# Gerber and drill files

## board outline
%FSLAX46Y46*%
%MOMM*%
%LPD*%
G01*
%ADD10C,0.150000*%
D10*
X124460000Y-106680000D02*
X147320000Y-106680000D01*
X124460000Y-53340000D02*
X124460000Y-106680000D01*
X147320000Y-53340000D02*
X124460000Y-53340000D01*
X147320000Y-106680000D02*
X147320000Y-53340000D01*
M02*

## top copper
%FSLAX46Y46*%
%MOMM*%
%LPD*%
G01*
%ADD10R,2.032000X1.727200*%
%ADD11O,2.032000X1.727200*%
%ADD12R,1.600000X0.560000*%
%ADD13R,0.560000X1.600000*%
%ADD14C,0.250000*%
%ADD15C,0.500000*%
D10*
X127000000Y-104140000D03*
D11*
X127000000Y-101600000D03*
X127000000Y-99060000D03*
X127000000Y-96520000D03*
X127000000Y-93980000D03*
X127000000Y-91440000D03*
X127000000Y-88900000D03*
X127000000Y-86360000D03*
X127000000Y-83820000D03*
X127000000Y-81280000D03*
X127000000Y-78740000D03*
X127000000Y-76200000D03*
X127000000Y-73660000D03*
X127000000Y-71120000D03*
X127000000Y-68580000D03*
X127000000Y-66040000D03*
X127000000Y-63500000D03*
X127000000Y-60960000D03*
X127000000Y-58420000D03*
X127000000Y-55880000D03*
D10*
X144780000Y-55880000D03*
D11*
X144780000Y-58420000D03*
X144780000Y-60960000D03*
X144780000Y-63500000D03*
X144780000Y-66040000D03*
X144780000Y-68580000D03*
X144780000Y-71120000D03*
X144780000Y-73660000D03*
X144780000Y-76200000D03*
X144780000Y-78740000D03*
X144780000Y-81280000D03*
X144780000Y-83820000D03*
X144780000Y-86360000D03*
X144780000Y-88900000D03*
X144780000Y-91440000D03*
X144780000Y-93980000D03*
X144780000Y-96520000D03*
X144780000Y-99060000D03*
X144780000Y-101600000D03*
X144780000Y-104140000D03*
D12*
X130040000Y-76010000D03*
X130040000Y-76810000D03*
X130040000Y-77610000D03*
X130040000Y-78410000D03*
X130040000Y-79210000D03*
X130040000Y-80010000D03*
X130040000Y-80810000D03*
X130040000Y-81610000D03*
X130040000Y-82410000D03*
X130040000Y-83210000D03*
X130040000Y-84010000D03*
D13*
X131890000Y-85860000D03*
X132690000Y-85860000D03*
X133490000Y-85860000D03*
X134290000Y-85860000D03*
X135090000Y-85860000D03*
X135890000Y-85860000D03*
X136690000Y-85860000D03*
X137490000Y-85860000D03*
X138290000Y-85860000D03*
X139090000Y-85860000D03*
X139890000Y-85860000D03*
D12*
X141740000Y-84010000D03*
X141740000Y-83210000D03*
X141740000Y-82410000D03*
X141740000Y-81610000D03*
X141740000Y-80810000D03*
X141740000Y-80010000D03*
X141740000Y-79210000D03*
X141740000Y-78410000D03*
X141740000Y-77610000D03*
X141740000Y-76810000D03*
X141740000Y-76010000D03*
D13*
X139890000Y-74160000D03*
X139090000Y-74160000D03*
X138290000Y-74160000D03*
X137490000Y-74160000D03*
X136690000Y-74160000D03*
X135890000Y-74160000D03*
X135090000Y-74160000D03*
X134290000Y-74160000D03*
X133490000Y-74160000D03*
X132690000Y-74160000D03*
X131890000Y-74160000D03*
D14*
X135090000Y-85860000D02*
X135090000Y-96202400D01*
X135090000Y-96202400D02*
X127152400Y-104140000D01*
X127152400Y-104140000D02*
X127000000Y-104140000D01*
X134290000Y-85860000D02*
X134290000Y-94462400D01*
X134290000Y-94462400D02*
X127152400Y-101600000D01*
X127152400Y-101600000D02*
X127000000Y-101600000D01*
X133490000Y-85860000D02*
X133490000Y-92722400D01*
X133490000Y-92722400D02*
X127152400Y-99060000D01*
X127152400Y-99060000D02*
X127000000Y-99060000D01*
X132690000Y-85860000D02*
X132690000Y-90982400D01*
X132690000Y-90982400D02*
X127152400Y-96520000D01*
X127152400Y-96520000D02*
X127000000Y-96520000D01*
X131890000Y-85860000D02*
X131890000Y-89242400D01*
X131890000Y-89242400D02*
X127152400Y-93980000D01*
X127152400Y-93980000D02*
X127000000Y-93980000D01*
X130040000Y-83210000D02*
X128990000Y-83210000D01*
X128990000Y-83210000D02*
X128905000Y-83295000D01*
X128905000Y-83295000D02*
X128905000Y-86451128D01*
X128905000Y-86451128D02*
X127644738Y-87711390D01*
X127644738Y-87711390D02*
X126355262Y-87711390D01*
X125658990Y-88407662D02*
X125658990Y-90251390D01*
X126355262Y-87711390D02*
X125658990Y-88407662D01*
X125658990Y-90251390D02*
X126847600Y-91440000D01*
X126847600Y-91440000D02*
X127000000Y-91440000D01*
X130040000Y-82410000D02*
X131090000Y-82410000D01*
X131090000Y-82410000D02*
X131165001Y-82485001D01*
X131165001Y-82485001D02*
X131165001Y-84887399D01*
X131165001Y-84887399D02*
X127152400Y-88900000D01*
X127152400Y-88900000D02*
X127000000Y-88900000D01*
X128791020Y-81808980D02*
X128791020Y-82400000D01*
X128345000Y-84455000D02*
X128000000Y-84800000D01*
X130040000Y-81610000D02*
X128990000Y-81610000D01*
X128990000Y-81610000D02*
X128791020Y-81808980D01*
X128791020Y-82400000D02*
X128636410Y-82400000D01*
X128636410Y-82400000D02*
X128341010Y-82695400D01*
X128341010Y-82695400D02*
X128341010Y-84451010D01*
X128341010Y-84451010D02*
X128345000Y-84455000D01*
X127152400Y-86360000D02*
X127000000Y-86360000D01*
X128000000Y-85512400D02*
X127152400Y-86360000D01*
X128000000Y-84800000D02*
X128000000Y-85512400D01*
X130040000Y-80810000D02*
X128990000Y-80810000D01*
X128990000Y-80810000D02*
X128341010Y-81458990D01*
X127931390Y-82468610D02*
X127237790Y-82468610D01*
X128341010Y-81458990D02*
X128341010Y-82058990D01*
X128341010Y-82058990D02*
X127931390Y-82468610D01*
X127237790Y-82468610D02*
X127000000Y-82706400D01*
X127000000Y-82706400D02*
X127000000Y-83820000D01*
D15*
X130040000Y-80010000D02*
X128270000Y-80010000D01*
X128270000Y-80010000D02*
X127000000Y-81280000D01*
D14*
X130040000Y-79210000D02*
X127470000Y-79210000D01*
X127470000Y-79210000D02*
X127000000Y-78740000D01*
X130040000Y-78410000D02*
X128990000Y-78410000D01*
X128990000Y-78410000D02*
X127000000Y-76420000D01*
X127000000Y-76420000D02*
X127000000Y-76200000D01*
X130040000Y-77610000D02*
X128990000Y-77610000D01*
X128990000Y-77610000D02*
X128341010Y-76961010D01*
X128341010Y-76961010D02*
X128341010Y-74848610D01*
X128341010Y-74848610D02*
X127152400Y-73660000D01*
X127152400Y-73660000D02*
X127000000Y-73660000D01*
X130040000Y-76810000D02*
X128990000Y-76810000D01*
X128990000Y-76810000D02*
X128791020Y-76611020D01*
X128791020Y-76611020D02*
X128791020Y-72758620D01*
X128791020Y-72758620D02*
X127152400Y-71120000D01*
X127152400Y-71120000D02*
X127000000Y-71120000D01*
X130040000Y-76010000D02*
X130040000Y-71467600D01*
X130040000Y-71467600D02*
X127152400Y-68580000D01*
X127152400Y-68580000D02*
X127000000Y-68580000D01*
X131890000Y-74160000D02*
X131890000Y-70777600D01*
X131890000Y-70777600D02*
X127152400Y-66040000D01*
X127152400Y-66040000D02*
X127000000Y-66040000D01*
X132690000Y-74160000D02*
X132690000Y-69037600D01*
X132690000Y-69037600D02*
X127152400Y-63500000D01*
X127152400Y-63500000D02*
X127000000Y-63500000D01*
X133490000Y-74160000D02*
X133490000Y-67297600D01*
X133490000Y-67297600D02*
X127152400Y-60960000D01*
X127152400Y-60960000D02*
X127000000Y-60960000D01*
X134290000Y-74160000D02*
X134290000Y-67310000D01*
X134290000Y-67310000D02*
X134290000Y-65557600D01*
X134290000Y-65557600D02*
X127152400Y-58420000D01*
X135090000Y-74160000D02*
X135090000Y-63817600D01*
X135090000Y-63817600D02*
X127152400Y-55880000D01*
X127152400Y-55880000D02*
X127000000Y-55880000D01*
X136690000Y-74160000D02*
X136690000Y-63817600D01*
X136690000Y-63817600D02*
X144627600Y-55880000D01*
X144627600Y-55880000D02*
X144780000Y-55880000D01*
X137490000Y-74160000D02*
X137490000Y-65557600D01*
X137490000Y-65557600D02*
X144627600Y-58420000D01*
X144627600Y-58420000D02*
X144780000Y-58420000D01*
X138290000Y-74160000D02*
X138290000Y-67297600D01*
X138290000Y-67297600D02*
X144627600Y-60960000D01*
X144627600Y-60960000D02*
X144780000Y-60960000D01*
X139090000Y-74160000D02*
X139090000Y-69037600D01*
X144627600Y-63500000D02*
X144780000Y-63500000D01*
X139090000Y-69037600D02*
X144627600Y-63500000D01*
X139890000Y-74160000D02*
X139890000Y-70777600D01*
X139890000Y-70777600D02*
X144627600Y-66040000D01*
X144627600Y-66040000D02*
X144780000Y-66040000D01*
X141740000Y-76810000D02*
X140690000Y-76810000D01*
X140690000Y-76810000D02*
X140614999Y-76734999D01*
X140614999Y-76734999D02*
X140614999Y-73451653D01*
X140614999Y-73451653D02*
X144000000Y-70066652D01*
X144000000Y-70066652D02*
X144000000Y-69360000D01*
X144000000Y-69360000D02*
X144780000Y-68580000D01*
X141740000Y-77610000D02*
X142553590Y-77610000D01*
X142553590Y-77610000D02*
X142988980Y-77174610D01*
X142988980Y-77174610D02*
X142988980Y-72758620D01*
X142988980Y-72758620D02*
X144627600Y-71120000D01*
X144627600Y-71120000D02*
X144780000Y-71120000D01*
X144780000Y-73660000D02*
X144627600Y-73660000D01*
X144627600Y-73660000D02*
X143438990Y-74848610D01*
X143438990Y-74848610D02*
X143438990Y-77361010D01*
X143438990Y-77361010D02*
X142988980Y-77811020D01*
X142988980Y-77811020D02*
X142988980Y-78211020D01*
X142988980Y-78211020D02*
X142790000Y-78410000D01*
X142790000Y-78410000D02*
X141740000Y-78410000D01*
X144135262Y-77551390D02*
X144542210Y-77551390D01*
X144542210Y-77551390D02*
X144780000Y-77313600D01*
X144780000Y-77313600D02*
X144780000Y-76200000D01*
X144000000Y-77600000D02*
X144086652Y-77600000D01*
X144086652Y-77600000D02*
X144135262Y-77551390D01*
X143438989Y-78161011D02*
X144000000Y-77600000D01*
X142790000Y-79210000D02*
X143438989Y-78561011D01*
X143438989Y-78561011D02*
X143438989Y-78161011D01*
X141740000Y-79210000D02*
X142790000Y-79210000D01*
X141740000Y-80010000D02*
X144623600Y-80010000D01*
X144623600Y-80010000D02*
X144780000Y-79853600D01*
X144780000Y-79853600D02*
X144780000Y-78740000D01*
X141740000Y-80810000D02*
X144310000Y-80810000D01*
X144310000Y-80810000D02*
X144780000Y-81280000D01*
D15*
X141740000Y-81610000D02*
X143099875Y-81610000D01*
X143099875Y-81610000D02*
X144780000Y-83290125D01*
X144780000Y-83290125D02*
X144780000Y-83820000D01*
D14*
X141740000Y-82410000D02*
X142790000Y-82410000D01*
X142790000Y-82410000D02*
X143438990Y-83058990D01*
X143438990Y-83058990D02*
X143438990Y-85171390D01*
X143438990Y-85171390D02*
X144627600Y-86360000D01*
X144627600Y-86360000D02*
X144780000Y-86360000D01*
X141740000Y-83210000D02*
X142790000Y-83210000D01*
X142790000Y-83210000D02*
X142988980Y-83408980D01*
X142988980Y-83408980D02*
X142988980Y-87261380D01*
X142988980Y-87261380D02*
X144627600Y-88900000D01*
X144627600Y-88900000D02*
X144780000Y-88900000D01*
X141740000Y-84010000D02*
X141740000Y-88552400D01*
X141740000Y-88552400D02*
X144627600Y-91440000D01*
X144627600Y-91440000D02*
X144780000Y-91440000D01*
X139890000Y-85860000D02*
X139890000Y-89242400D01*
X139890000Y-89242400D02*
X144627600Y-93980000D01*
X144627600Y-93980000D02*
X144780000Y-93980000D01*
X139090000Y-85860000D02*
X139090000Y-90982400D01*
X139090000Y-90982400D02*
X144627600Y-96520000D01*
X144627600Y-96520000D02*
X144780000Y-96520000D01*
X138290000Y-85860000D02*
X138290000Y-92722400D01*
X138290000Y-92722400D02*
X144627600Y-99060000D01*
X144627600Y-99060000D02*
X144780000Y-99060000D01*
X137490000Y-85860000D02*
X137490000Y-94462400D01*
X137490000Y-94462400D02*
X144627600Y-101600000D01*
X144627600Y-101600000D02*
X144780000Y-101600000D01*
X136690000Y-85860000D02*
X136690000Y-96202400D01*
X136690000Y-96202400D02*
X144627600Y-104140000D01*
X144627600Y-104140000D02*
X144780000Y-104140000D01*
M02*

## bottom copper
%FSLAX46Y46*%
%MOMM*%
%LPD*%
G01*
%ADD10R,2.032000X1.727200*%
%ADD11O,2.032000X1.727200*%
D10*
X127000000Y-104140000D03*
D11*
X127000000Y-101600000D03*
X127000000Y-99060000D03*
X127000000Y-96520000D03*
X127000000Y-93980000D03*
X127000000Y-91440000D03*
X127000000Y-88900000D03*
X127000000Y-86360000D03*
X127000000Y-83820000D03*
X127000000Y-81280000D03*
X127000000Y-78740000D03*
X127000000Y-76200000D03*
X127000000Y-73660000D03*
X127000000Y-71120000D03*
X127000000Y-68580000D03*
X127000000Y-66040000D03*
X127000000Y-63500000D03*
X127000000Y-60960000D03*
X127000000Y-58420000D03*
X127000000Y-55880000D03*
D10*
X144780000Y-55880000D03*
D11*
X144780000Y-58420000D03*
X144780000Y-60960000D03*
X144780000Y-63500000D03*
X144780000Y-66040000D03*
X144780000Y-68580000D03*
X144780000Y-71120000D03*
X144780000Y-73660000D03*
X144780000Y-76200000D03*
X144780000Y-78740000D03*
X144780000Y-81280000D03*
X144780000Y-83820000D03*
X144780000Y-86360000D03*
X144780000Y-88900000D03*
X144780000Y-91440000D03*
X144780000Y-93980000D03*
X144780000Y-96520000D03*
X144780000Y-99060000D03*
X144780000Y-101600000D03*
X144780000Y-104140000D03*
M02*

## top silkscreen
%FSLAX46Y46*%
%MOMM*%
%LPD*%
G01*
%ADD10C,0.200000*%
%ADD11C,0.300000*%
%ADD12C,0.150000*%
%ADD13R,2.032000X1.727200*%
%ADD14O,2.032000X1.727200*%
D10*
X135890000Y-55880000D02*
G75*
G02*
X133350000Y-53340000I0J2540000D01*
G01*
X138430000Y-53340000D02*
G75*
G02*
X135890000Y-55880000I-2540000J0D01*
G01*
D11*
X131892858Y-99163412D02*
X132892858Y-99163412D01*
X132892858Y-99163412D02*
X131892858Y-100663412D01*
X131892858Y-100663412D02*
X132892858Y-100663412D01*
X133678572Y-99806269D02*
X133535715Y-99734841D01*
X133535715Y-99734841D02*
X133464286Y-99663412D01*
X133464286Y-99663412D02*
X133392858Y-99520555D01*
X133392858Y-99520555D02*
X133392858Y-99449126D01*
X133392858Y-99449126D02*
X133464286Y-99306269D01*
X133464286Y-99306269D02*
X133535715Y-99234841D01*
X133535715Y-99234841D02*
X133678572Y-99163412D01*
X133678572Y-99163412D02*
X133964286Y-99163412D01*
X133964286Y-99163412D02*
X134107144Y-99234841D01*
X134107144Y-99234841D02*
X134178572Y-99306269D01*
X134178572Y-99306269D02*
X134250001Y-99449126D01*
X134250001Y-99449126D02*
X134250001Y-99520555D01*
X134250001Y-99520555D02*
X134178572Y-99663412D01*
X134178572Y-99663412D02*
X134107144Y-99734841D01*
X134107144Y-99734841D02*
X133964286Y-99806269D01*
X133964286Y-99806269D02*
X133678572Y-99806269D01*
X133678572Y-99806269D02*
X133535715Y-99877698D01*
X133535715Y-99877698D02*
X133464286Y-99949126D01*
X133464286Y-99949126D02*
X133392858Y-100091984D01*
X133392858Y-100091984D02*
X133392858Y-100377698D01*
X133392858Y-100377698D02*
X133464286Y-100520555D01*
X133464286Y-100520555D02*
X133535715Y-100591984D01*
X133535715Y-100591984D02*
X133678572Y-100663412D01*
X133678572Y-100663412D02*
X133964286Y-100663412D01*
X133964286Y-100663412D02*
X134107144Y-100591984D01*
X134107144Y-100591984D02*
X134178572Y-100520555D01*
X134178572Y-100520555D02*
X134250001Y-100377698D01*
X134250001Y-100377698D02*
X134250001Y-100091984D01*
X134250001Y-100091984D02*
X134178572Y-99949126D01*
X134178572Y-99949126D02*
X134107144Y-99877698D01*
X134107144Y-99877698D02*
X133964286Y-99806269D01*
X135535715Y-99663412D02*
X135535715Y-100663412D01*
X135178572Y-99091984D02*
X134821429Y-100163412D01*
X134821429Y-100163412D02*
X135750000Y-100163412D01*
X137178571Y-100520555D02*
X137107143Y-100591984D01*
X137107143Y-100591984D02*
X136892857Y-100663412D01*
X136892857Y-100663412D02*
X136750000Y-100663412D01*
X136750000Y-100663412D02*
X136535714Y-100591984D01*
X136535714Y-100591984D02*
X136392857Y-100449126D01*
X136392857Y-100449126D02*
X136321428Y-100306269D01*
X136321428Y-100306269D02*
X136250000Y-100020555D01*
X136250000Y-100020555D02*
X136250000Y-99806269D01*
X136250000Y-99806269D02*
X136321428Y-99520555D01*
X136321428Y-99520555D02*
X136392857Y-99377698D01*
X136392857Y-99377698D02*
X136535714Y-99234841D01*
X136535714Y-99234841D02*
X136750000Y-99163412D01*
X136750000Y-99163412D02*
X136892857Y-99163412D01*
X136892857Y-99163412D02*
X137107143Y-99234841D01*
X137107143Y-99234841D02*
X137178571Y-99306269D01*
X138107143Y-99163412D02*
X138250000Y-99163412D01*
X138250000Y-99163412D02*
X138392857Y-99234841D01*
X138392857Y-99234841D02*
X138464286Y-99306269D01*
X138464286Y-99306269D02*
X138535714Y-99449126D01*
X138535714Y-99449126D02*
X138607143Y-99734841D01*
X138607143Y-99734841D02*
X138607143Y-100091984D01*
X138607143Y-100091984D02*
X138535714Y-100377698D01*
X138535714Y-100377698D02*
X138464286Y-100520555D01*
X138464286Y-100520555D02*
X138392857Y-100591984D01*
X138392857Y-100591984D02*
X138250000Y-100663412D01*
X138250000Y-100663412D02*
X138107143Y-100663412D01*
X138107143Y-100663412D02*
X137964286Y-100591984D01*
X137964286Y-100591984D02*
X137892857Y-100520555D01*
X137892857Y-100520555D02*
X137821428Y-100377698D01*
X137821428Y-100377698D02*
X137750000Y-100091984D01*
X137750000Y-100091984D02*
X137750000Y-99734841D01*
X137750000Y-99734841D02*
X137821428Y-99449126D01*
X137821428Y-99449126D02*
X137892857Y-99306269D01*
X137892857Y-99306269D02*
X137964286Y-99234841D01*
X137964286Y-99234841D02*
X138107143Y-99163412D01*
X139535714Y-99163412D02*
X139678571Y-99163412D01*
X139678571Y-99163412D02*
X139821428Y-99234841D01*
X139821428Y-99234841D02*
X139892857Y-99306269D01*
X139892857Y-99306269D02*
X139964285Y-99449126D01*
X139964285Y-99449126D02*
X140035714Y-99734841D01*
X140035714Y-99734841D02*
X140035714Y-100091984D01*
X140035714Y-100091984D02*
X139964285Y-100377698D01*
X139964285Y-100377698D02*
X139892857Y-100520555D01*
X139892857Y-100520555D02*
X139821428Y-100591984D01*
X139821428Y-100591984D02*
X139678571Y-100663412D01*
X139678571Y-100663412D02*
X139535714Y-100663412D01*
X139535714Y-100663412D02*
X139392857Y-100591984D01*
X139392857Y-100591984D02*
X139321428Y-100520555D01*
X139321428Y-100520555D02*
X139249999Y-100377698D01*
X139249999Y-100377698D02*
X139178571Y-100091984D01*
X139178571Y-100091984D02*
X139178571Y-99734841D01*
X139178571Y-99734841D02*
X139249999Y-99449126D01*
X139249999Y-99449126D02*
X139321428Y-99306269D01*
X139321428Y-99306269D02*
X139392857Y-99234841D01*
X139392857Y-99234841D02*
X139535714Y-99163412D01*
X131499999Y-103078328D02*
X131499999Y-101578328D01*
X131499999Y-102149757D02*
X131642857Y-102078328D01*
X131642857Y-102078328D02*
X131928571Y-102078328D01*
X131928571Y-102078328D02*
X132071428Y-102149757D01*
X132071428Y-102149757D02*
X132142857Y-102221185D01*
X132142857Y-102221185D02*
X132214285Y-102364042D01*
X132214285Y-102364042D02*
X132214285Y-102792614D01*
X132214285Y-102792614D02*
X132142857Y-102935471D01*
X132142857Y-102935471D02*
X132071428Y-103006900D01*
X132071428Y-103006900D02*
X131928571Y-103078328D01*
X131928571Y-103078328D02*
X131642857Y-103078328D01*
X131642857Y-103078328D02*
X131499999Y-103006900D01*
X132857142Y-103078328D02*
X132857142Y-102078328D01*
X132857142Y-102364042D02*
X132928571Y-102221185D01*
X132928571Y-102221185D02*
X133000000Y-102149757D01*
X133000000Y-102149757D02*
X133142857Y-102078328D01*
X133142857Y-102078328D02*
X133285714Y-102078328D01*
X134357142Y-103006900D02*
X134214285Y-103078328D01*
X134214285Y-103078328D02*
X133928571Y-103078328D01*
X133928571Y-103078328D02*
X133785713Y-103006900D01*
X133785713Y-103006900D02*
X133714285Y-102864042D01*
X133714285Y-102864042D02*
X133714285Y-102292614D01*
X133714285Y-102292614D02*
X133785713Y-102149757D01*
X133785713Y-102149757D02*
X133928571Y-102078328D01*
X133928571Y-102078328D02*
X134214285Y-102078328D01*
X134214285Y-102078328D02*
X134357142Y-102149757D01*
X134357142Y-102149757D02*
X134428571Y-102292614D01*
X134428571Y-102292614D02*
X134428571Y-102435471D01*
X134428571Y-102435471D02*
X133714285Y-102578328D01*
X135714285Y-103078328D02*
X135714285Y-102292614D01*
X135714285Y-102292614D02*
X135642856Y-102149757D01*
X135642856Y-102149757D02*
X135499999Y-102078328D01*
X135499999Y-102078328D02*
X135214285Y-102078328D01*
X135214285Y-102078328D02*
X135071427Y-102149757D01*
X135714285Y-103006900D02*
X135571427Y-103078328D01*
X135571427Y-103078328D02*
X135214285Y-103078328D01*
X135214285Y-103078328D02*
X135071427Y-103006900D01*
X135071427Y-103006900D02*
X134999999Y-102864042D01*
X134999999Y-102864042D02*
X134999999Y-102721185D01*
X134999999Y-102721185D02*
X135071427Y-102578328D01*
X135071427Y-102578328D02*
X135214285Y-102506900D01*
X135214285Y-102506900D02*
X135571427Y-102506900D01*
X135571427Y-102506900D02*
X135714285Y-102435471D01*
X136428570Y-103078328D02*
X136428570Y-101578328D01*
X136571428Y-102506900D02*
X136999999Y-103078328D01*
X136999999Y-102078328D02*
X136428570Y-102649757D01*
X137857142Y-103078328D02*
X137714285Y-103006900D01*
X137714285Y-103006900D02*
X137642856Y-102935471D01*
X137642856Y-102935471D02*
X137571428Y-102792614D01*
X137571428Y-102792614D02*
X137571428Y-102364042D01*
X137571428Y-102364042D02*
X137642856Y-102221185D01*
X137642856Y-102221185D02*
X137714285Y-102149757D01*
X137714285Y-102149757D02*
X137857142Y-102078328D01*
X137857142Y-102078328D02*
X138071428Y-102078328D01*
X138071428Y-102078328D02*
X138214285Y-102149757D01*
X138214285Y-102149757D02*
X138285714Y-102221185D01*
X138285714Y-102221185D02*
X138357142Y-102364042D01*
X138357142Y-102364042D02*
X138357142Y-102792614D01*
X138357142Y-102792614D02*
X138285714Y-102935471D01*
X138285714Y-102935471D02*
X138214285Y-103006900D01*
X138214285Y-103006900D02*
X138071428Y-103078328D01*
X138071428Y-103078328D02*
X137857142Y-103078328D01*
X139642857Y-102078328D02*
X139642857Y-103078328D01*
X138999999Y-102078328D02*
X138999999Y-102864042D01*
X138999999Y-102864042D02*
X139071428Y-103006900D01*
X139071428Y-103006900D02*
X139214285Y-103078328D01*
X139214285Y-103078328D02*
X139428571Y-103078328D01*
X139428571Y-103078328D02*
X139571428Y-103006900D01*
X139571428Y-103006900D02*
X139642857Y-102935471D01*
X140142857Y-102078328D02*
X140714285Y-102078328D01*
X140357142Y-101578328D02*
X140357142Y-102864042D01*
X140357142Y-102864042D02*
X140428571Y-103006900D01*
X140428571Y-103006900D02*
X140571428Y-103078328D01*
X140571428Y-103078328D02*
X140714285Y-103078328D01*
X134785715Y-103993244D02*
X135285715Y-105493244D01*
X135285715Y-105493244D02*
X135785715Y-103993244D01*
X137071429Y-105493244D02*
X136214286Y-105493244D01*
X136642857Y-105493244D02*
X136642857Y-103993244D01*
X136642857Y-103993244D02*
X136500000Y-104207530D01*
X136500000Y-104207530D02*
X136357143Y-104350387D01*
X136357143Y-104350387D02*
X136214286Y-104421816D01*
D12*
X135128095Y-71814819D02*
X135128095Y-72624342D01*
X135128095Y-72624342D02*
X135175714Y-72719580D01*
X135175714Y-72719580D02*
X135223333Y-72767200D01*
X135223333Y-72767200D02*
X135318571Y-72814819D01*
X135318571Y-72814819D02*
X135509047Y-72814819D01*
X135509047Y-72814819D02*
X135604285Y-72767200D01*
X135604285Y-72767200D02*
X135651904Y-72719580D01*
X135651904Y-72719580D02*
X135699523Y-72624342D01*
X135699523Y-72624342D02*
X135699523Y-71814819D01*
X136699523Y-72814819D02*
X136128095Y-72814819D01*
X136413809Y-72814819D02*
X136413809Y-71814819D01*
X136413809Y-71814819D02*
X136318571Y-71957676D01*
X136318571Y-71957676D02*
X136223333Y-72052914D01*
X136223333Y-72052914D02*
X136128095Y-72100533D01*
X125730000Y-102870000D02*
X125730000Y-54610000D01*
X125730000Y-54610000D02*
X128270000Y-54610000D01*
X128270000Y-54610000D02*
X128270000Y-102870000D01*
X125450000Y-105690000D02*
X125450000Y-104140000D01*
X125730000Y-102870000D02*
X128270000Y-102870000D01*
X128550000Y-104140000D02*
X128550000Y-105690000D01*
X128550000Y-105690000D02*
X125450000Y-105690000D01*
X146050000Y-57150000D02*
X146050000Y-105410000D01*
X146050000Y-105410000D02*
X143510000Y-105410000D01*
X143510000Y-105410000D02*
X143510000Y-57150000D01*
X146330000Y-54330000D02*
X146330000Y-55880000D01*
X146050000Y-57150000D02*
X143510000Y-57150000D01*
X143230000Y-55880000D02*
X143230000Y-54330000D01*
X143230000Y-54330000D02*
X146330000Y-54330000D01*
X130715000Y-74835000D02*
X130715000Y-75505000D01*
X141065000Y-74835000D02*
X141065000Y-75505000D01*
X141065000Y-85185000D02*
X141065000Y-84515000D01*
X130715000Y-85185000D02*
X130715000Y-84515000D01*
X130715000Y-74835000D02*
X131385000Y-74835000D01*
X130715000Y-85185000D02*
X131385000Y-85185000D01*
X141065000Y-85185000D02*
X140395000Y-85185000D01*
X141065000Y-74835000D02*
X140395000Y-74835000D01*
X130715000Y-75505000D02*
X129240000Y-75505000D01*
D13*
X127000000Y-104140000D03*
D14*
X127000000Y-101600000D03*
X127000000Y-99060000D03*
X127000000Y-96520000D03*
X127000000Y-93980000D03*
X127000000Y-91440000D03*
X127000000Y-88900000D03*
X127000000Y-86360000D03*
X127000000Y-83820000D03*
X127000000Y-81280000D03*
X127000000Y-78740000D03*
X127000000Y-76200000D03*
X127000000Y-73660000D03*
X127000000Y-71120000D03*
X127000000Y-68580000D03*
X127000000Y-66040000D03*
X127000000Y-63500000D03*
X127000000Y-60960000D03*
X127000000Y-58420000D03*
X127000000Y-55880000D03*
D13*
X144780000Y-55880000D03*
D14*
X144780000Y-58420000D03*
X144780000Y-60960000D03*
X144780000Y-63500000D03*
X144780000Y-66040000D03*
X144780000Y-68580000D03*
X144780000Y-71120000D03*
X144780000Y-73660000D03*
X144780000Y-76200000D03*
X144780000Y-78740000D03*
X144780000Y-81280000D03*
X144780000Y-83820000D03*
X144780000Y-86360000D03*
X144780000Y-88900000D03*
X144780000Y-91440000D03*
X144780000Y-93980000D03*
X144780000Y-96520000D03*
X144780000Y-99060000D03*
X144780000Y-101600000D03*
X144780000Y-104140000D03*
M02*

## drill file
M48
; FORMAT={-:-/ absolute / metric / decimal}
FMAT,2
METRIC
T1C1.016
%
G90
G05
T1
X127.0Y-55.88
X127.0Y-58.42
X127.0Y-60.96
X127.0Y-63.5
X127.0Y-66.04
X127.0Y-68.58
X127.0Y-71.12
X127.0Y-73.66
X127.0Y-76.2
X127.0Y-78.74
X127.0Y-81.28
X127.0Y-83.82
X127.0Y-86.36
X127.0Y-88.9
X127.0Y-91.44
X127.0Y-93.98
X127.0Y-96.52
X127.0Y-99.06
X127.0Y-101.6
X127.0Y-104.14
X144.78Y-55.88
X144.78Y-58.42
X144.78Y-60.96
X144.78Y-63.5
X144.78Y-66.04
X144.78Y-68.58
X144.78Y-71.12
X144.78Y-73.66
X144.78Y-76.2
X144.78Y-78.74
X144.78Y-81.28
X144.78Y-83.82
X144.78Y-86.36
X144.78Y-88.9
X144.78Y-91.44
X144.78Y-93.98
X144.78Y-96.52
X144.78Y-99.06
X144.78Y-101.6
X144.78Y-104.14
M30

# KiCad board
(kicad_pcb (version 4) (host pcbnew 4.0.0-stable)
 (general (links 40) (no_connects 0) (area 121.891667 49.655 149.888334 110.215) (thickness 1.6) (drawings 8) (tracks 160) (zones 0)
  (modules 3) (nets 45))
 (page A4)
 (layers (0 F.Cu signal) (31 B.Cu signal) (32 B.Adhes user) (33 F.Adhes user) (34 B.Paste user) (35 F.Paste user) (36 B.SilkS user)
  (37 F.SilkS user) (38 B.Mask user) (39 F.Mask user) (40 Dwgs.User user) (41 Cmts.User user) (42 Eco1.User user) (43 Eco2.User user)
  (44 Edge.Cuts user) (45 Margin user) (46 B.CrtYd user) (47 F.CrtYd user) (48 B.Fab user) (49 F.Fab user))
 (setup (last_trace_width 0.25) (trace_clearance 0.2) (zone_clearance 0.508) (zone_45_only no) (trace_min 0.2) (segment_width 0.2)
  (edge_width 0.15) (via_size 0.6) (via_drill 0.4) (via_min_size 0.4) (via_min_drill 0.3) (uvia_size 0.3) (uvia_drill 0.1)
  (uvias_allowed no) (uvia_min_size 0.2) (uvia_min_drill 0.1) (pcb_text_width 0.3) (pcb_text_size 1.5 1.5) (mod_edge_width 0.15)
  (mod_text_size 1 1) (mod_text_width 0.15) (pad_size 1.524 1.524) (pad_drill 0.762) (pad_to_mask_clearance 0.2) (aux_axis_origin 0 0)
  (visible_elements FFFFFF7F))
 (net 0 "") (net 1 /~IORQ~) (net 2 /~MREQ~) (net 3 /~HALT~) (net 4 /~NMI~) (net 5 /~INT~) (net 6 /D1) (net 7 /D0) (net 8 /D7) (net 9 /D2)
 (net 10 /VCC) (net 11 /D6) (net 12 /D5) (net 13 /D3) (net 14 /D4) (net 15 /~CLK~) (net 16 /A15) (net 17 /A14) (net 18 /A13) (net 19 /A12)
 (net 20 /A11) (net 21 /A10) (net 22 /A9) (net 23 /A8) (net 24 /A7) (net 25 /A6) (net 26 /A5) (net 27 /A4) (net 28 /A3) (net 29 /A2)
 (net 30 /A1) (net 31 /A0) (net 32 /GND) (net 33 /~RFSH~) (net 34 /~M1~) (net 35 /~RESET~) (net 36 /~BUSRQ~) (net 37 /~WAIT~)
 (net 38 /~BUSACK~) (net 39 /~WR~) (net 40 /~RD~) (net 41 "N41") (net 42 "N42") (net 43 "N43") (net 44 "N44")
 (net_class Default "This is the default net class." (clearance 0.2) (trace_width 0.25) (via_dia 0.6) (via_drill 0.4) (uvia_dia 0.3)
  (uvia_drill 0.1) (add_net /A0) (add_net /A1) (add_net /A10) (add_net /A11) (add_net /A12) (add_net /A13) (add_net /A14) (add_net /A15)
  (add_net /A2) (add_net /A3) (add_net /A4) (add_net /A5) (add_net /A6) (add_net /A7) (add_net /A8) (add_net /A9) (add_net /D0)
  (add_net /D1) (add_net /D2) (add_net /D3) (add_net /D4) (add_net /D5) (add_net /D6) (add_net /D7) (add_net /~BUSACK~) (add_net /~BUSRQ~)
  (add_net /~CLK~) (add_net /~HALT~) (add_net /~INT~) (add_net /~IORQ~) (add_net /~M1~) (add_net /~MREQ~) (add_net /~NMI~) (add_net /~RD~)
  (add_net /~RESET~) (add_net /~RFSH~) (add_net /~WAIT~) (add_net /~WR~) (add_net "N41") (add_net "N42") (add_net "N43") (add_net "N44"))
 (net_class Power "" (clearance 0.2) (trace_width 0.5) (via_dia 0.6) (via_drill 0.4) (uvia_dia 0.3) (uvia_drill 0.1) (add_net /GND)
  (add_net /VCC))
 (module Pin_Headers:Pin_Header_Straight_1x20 (layer F.Cu) (at 127 104.14 180)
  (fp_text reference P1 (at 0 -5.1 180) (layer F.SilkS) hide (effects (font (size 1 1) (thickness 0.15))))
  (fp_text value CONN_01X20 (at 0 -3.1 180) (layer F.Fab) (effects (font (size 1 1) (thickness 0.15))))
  (fp_line (start 1.27 1.27) (end 1.27 49.53) (layer F.SilkS) (width 0.15))
  (fp_line (start 1.27 49.53) (end -1.27 49.53) (layer F.SilkS) (width 0.15))
  (fp_line (start -1.27 49.53) (end -1.27 1.27) (layer F.SilkS) (width 0.15))
  (fp_line (start 1.55 -1.55) (end 1.55 0) (layer F.SilkS) (width 0.15))
  (fp_line (start 1.27 1.27) (end -1.27 1.27) (layer F.SilkS) (width 0.15))
  (fp_line (start -1.55 0) (end -1.55 -1.55) (layer F.SilkS) (width 0.15))
  (fp_line (start -1.55 -1.55) (end 1.55 -1.55) (layer F.SilkS) (width 0.15))
  (pad 1 thru_hole rect (at 0 0 180) (size 2.032 1.7272) (drill 1.016) (layers *.Cu *.Mask F.SilkS) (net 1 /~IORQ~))
  (pad 2 thru_hole oval (at 0 2.54 180) (size 2.032 1.7272) (drill 1.016) (layers *.Cu *.Mask F.SilkS) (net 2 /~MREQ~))
  (pad 3 thru_hole oval (at 0 5.08 180) (size 2.032 1.7272) (drill 1.016) (layers *.Cu *.Mask F.SilkS) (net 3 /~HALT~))
  (pad 4 thru_hole oval (at 0 7.62 180) (size 2.032 1.7272) (drill 1.016) (layers *.Cu *.Mask F.SilkS) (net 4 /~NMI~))
  (pad 5 thru_hole oval (at 0 10.16 180) (size 2.032 1.7272) (drill 1.016) (layers *.Cu *.Mask F.SilkS) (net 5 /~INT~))
  (pad 6 thru_hole oval (at 0 12.7 180) (size 2.032 1.7272) (drill 1.016) (layers *.Cu *.Mask F.SilkS) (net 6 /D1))
  (pad 7 thru_hole oval (at 0 15.24 180) (size 2.032 1.7272) (drill 1.016) (layers *.Cu *.Mask F.SilkS) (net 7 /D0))
  (pad 8 thru_hole oval (at 0 17.78 180) (size 2.032 1.7272) (drill 1.016) (layers *.Cu *.Mask F.SilkS) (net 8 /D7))
  (pad 9 thru_hole oval (at 0 20.32 180) (size 2.032 1.7272) (drill 1.016) (layers *.Cu *.Mask F.SilkS) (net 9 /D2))
  (pad 10 thru_hole oval (at 0 22.86 180) (size 2.032 1.7272) (drill 1.016) (layers *.Cu *.Mask F.SilkS) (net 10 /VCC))
  (pad 11 thru_hole oval (at 0 25.4 180) (size 2.032 1.7272) (drill 1.016) (layers *.Cu *.Mask F.SilkS) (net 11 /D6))
  (pad 12 thru_hole oval (at 0 27.94 180) (size 2.032 1.7272) (drill 1.016) (layers *.Cu *.Mask F.SilkS) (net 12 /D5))
  (pad 13 thru_hole oval (at 0 30.48 180) (size 2.032 1.7272) (drill 1.016) (layers *.Cu *.Mask F.SilkS) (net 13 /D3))
  (pad 14 thru_hole oval (at 0 33.02 180) (size 2.032 1.7272) (drill 1.016) (layers *.Cu *.Mask F.SilkS) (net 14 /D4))
  (pad 15 thru_hole oval (at 0 35.56 180) (size 2.032 1.7272) (drill 1.016) (layers *.Cu *.Mask F.SilkS) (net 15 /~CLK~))
  (pad 16 thru_hole oval (at 0 38.1 180) (size 2.032 1.7272) (drill 1.016) (layers *.Cu *.Mask F.SilkS) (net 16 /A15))
  (pad 17 thru_hole oval (at 0 40.64 180) (size 2.032 1.7272) (drill 1.016) (layers *.Cu *.Mask F.SilkS) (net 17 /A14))
  (pad 18 thru_hole oval (at 0 43.18 180) (size 2.032 1.7272) (drill 1.016) (layers *.Cu *.Mask F.SilkS) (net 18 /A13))
  (pad 19 thru_hole oval (at 0 45.72 180) (size 2.032 1.7272) (drill 1.016) (layers *.Cu *.Mask F.SilkS) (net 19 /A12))
  (pad 20 thru_hole oval (at 0 48.26 180) (size 2.032 1.7272) (drill 1.016) (layers *.Cu *.Mask F.SilkS) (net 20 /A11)))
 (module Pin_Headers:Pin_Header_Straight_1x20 (layer F.Cu) (at 144.78 55.88)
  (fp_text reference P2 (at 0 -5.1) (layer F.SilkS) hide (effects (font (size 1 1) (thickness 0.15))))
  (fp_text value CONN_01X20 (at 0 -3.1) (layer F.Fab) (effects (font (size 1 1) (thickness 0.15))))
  (fp_line (start 1.27 1.27) (end 1.27 49.53) (layer F.SilkS) (width 0.15))
  (fp_line (start 1.27 49.53) (end -1.27 49.53) (layer F.SilkS) (width 0.15))
  (fp_line (start -1.27 49.53) (end -1.27 1.27) (layer F.SilkS) (width 0.15))
  (fp_line (start 1.55 -1.55) (end 1.55 0) (layer F.SilkS) (width 0.15))
  (fp_line (start 1.27 1.27) (end -1.27 1.27) (layer F.SilkS) (width 0.15))
  (fp_line (start -1.55 0) (end -1.55 -1.55) (layer F.SilkS) (width 0.15))
  (fp_line (start -1.55 -1.55) (end 1.55 -1.55) (layer F.SilkS) (width 0.15))
  (pad 1 thru_hole rect (at 0 0) (size 2.032 1.7272) (drill 1.016) (layers *.Cu *.Mask F.SilkS) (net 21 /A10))
  (pad 2 thru_hole oval (at 0 2.54) (size 2.032 1.7272) (drill 1.016) (layers *.Cu *.Mask F.SilkS) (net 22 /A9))
  (pad 3 thru_hole oval (at 0 5.08) (size 2.032 1.7272) (drill 1.016) (layers *.Cu *.Mask F.SilkS) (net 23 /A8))
  (pad 4 thru_hole oval (at 0 7.62) (size 2.032 1.7272) (drill 1.016) (layers *.Cu *.Mask F.SilkS) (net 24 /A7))
  (pad 5 thru_hole oval (at 0 10.16) (size 2.032 1.7272) (drill 1.016) (layers *.Cu *.Mask F.SilkS) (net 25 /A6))
  (pad 6 thru_hole oval (at 0 12.7) (size 2.032 1.7272) (drill 1.016) (layers *.Cu *.Mask F.SilkS) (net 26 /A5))
  (pad 7 thru_hole oval (at 0 15.24) (size 2.032 1.7272) (drill 1.016) (layers *.Cu *.Mask F.SilkS) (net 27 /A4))
  (pad 8 thru_hole oval (at 0 17.78) (size 2.032 1.7272) (drill 1.016) (layers *.Cu *.Mask F.SilkS) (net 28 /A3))
  (pad 9 thru_hole oval (at 0 20.32) (size 2.032 1.7272) (drill 1.016) (layers *.Cu *.Mask F.SilkS) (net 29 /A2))
  (pad 10 thru_hole oval (at 0 22.86) (size 2.032 1.7272) (drill 1.016) (layers *.Cu *.Mask F.SilkS) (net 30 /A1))
  (pad 11 thru_hole oval (at 0 25.4) (size 2.032 1.7272) (drill 1.016) (layers *.Cu *.Mask F.SilkS) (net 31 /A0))
  (pad 12 thru_hole oval (at 0 27.94) (size 2.032 1.7272) (drill 1.016) (layers *.Cu *.Mask F.SilkS) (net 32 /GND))
  (pad 13 thru_hole oval (at 0 30.48) (size 2.032 1.7272) (drill 1.016) (layers *.Cu *.Mask F.SilkS) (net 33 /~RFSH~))
  (pad 14 thru_hole oval (at 0 33.02) (size 2.032 1.7272) (drill 1.016) (layers *.Cu *.Mask F.SilkS) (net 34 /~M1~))
  (pad 15 thru_hole oval (at 0 35.56) (size 2.032 1.7272) (drill 1.016) (layers *.Cu *.Mask F.SilkS) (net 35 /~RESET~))
  (pad 16 thru_hole oval (at 0 38.1) (size 2.032 1.7272) (drill 1.016) (layers *.Cu *.Mask F.SilkS) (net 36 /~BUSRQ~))
  (pad 17 thru_hole oval (at 0 40.64) (size 2.032 1.7272) (drill 1.016) (layers *.Cu *.Mask F.SilkS) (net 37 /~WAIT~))
  (pad 18 thru_hole oval (at 0 43.18) (size 2.032 1.7272) (drill 1.016) (layers *.Cu *.Mask F.SilkS) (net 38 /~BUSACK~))
  (pad 19 thru_hole oval (at 0 45.72) (size 2.032 1.7272) (drill 1.016) (layers *.Cu *.Mask F.SilkS) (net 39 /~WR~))
  (pad 20 thru_hole oval (at 0 48.26) (size 2.032 1.7272) (drill 1.016) (layers *.Cu *.Mask F.SilkS) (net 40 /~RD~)))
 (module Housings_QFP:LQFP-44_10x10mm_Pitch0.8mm (layer F.Cu) (at 135.89 80.01)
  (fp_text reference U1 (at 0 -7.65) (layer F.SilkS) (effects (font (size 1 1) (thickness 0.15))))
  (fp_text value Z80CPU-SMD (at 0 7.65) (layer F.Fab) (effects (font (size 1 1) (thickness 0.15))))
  (fp_line (start -5.175 -5.175) (end -5.175 -4.505) (layer F.SilkS) (width 0.15))
  (fp_line (start 5.175 -5.175) (end 5.175 -4.505) (layer F.SilkS) (width 0.15))
  (fp_line (start 5.175 5.175) (end 5.175 4.505) (layer F.SilkS) (width 0.15))
  (fp_line (start -5.175 5.175) (end -5.175 4.505) (layer F.SilkS) (width 0.15))
  (fp_line (start -5.175 -5.175) (end -4.505 -5.175) (layer F.SilkS) (width 0.15))
  (fp_line (start -5.175 5.175) (end -4.505 5.175) (layer F.SilkS) (width 0.15))
  (fp_line (start 5.175 5.175) (end 4.505 5.175) (layer F.SilkS) (width 0.15))
  (fp_line (start 5.175 -5.175) (end 4.505 -5.175) (layer F.SilkS) (width 0.15))
  (fp_line (start -5.175 -4.505) (end -6.65 -4.505) (layer F.SilkS) (width 0.15))
  (pad 1 smd rect (at -5.85 -4) (size 1.6 0.56) (layers F.Cu F.Paste F.Mask) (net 15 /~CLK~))
  (pad 2 smd rect (at -5.85 -3.2) (size 1.6 0.56) (layers F.Cu F.Paste F.Mask) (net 14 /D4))
  (pad 3 smd rect (at -5.85 -2.4) (size 1.6 0.56) (layers F.Cu F.Paste F.Mask) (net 13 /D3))
  (pad 4 smd rect (at -5.85 -1.6) (size 1.6 0.56) (layers F.Cu F.Paste F.Mask) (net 12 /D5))
  (pad 5 smd rect (at -5.85 -0.8) (size 1.6 0.56) (layers F.Cu F.Paste F.Mask) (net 11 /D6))
  (pad 6 smd rect (at -5.85 0) (size 1.6 0.56) (layers F.Cu F.Paste F.Mask) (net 10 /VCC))
  (pad 7 smd rect (at -5.85 0.8) (size 1.6 0.56) (layers F.Cu F.Paste F.Mask) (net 9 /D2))
  (pad 8 smd rect (at -5.85 1.6) (size 1.6 0.56) (layers F.Cu F.Paste F.Mask) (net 8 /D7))
  (pad 9 smd rect (at -5.85 2.4) (size 1.6 0.56) (layers F.Cu F.Paste F.Mask) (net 7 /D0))
  (pad 10 smd rect (at -5.85 3.2) (size 1.6 0.56) (layers F.Cu F.Paste F.Mask) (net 6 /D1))
  (pad 11 smd rect (at -5.85 4) (size 1.6 0.56) (layers F.Cu F.Paste F.Mask) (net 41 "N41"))
  (pad 12 smd rect (at -4 5.85 90) (size 1.6 0.56) (layers F.Cu F.Paste F.Mask) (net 5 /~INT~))
  (pad 13 smd rect (at -3.2 5.85 90) (size 1.6 0.56) (layers F.Cu F.Paste F.Mask) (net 4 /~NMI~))
  (pad 14 smd rect (at -2.4 5.85 90) (size 1.6 0.56) (layers F.Cu F.Paste F.Mask) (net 3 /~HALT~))
  (pad 15 smd rect (at -1.6 5.85 90) (size 1.6 0.56) (layers F.Cu F.Paste F.Mask) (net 2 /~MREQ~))
  (pad 16 smd rect (at -0.8 5.85 90) (size 1.6 0.56) (layers F.Cu F.Paste F.Mask) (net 1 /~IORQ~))
  (pad 17 smd rect (at 0 5.85 90) (size 1.6 0.56) (layers F.Cu F.Paste F.Mask) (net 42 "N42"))
  (pad 18 smd rect (at 0.8 5.85 90) (size 1.6 0.56) (layers F.Cu F.Paste F.Mask) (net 40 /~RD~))
  (pad 19 smd rect (at 1.6 5.85 90) (size 1.6 0.56) (layers F.Cu F.Paste F.Mask) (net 39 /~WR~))
  (pad 20 smd rect (at 2.4 5.85 90) (size 1.6 0.56) (layers F.Cu F.Paste F.Mask) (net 38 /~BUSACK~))
  (pad 21 smd rect (at 3.2 5.85 90) (size 1.6 0.56) (layers F.Cu F.Paste F.Mask) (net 37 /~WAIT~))
  (pad 22 smd rect (at 4 5.85 90) (size 1.6 0.56) (layers F.Cu F.Paste F.Mask) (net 36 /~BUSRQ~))
  (pad 23 smd rect (at 5.85 4) (size 1.6 0.56) (layers F.Cu F.Paste F.Mask) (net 35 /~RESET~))
  (pad 24 smd rect (at 5.85 3.2) (size 1.6 0.56) (layers F.Cu F.Paste F.Mask) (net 34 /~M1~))
  (pad 25 smd rect (at 5.85 2.4) (size 1.6 0.56) (layers F.Cu F.Paste F.Mask) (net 33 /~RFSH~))
  (pad 26 smd rect (at 5.85 1.6) (size 1.6 0.56) (layers F.Cu F.Paste F.Mask) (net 32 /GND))
  (pad 27 smd rect (at 5.85 0.8) (size 1.6 0.56) (layers F.Cu F.Paste F.Mask) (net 31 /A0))
  (pad 28 smd rect (at 5.85 0) (size 1.6 0.56) (layers F.Cu F.Paste F.Mask) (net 30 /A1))
  (pad 29 smd rect (at 5.85 -0.8) (size 1.6 0.56) (layers F.Cu F.Paste F.Mask) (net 29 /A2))
  (pad 30 smd rect (at 5.85 -1.6) (size 1.6 0.56) (layers F.Cu F.Paste F.Mask) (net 28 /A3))
  (pad 31 smd rect (at 5.85 -2.4) (size 1.6 0.56) (layers F.Cu F.Paste F.Mask) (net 27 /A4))
  (pad 32 smd rect (at 5.85 -3.2) (size 1.6 0.56) (layers F.Cu F.Paste F.Mask) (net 26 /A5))
  (pad 33 smd rect (at 5.85 -4) (size 1.6 0.56) (layers F.Cu F.Paste F.Mask) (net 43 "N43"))
  (pad 34 smd rect (at 4 -5.85 90) (size 1.6 0.56) (layers F.Cu F.Paste F.Mask) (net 25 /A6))
  (pad 35 smd rect (at 3.2 -5.85 90) (size 1.6 0.56) (layers F.Cu F.Paste F.Mask) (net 24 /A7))
  (pad 36 smd rect (at 2.4 -5.85 90) (size 1.6 0.56) (layers F.Cu F.Paste F.Mask) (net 23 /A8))
  (pad 37 smd rect (at 1.6 -5.85 90) (size 1.6 0.56) (layers F.Cu F.Paste F.Mask) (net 22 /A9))
  (pad 38 smd rect (at 0.8 -5.85 90) (size 1.6 0.56) (layers F.Cu F.Paste F.Mask) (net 21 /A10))
  (pad 39 smd rect (at 0 -5.85 90) (size 1.6 0.56) (layers F.Cu F.Paste F.Mask) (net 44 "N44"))
  (pad 40 smd rect (at -0.8 -5.85 90) (size 1.6 0.56) (layers F.Cu F.Paste F.Mask) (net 20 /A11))
  (pad 41 smd rect (at -1.6 -5.85 90) (size 1.6 0.56) (layers F.Cu F.Paste F.Mask) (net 19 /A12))
  (pad 42 smd rect (at -2.4 -5.85 90) (size 1.6 0.56) (layers F.Cu F.Paste F.Mask) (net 18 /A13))
  (pad 43 smd rect (at -3.2 -5.85 90) (size 1.6 0.56) (layers F.Cu F.Paste F.Mask) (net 17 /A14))
  (pad 44 smd rect (at -4 -5.85 90) (size 1.6 0.56) (layers F.Cu F.Paste F.Mask) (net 16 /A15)))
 (gr_arc (start 135.89 53.34) (end 135.89 55.88) (angle 90) (layer F.SilkS) (width 0.2))
 (gr_arc (start 135.89 53.34) (end 138.43 53.34) (angle 90) (layer F.SilkS) (width 0.2))
 (gr_line (start 124.46 106.68) (end 147.32 106.68) (layer Edge.Cuts) (width 0.15))
 (gr_line (start 124.46 53.34) (end 124.46 106.68) (layer Edge.Cuts) (width 0.15))
 (gr_line (start 147.32 53.34) (end 124.46 53.34) (layer Edge.Cuts) (width 0.15))
 (gr_line (start 147.32 106.68) (end 147.32 53.34) (layer Edge.Cuts) (width 0.15))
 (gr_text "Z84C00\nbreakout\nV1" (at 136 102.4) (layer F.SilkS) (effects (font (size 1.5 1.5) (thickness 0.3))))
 (segment (start 135.09 85.86) (end 135.09 96.2024) (width 0.25) (layer F.Cu) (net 1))
 (segment (start 135.09 96.2024) (end 127.1524 104.14) (width 0.25) (layer F.Cu) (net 1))
 (segment (start 127.1524 104.14) (end 127 104.14) (width 0.25) (layer F.Cu) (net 1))
 (segment (start 134.29 85.86) (end 134.29 94.4624) (width 0.25) (layer F.Cu) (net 2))
 (segment (start 134.29 94.4624) (end 127.1524 101.6) (width 0.25) (layer F.Cu) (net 2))
 (segment (start 127.1524 101.6) (end 127 101.6) (width 0.25) (layer F.Cu) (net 2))
 (segment (start 133.49 85.86) (end 133.49 92.7224) (width 0.25) (layer F.Cu) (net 3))
 (segment (start 133.49 92.7224) (end 127.1524 99.06) (width 0.25) (layer F.Cu) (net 3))
 (segment (start 127.1524 99.06) (end 127 99.06) (width 0.25) (layer F.Cu) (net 3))
 (segment (start 132.69 85.86) (end 132.69 90.9824) (width 0.25) (layer F.Cu) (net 4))
 (segment (start 132.69 90.9824) (end 127.1524 96.52) (width 0.25) (layer F.Cu) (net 4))
 (segment (start 127.1524 96.52) (end 127 96.52) (width 0.25) (layer F.Cu) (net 4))
 (segment (start 131.89 85.86) (end 131.89 89.2424) (width 0.25) (layer F.Cu) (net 5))
 (segment (start 131.89 89.2424) (end 127.1524 93.98) (width 0.25) (layer F.Cu) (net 5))
 (segment (start 127.1524 93.98) (end 127 93.98) (width 0.25) (layer F.Cu) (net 5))
 (segment (start 130.04 83.21) (end 128.99 83.21) (width 0.25) (layer F.Cu) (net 6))
 (segment (start 128.99 83.21) (end 128.905 83.295) (width 0.25) (layer F.Cu) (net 6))
 (segment (start 128.905 83.295) (end 128.905 86.451128) (width 0.25) (layer F.Cu) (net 6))
 (segment (start 128.905 86.451128) (end 127.644738 87.71139) (width 0.25) (layer F.Cu) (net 6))
 (segment (start 127.644738 87.71139) (end 126.355262 87.71139) (width 0.25) (layer F.Cu) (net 6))
 (segment (start 125.65899 88.407662) (end 125.65899 90.25139) (width 0.25) (layer F.Cu) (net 6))
 (segment (start 126.355262 87.71139) (end 125.65899 88.407662) (width 0.25) (layer F.Cu) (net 6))
 (segment (start 125.65899 90.25139) (end 126.8476 91.44) (width 0.25) (layer F.Cu) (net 6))
 (segment (start 126.8476 91.44) (end 127 91.44) (width 0.25) (layer F.Cu) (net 6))
 (segment (start 130.04 82.41) (end 131.09 82.41) (width 0.25) (layer F.Cu) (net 7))
 (segment (start 131.09 82.41) (end 131.165001 82.485001) (width 0.25) (layer F.Cu) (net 7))
 (segment (start 131.165001 82.485001) (end 131.165001 84.887399) (width 0.25) (layer F.Cu) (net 7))
 (segment (start 131.165001 84.887399) (end 127.1524 88.9) (width 0.25) (layer F.Cu) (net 7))
 (segment (start 127.1524 88.9) (end 127 88.9) (width 0.25) (layer F.Cu) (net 7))
 (segment (start 128.79102 81.80898) (end 128.79102 82.4) (width 0.25) (layer F.Cu) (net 8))
 (segment (start 128.345 84.455) (end 128 84.8) (width 0.25) (layer F.Cu) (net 8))
 (segment (start 130.04 81.61) (end 128.99 81.61) (width 0.25) (layer F.Cu) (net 8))
 (segment (start 128.99 81.61) (end 128.79102 81.80898) (width 0.25) (layer F.Cu) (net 8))
 (segment (start 128.79102 82.4) (end 128.63641 82.4) (width 0.25) (layer F.Cu) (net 8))
 (segment (start 128.63641 82.4) (end 128.34101 82.6954) (width 0.25) (layer F.Cu) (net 8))
 (segment (start 128.34101 82.6954) (end 128.34101 84.45101) (width 0.25) (layer F.Cu) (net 8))
 (segment (start 128.34101 84.45101) (end 128.345 84.455) (width 0.25) (layer F.Cu) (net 8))
 (segment (start 127.1524 86.36) (end 127 86.36) (width 0.25) (layer F.Cu) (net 8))
 (segment (start 128 85.5124) (end 127.1524 86.36) (width 0.25) (layer F.Cu) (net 8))
 (segment (start 128 84.8) (end 128 85.5124) (width 0.25) (layer F.Cu) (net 8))
 (segment (start 130.04 80.81) (end 128.99 80.81) (width 0.25) (layer F.Cu) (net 9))
 (segment (start 128.99 80.81) (end 128.34101 81.45899) (width 0.25) (layer F.Cu) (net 9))
 (segment (start 127.93139 82.46861) (end 127.23779 82.46861) (width 0.25) (layer F.Cu) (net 9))
 (segment (start 128.34101 81.45899) (end 128.34101 82.05899) (width 0.25) (layer F.Cu) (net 9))
 (segment (start 128.34101 82.05899) (end 127.93139 82.46861) (width 0.25) (layer F.Cu) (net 9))
 (segment (start 127.23779 82.46861) (end 127 82.7064) (width 0.25) (layer F.Cu) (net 9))
 (segment (start 127 82.7064) (end 127 83.82) (width 0.25) (layer F.Cu) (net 9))
 (segment (start 130.04 80.01) (end 128.27 80.01) (width 0.5) (layer F.Cu) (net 10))
 (segment (start 128.27 80.01) (end 127 81.28) (width 0.5) (layer F.Cu) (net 10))
 (segment (start 130.04 79.21) (end 127.47 79.21) (width 0.25) (layer F.Cu) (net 11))
 (segment (start 127.47 79.21) (end 127 78.74) (width 0.25) (layer F.Cu) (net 11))
 (segment (start 130.04 78.41) (end 128.99 78.41) (width 0.25) (layer F.Cu) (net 12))
 (segment (start 128.99 78.41) (end 127 76.42) (width 0.25) (layer F.Cu) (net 12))
 (segment (start 127 76.42) (end 127 76.2) (width 0.25) (layer F.Cu) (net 12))
 (segment (start 130.04 77.61) (end 128.99 77.61) (width 0.25) (layer F.Cu) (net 13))
 (segment (start 128.99 77.61) (end 128.34101 76.96101) (width 0.25) (layer F.Cu) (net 13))
 (segment (start 128.34101 76.96101) (end 128.34101 74.84861) (width 0.25) (layer F.Cu) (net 13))
 (segment (start 128.34101 74.84861) (end 127.1524 73.66) (width 0.25) (layer F.Cu) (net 13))
 (segment (start 127.1524 73.66) (end 127 73.66) (width 0.25) (layer F.Cu) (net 13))
 (segment (start 130.04 76.81) (end 128.99 76.81) (width 0.25) (layer F.Cu) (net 14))
 (segment (start 128.99 76.81) (end 128.79102 76.61102) (width 0.25) (layer F.Cu) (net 14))
 (segment (start 128.79102 76.61102) (end 128.79102 72.75862) (width 0.25) (layer F.Cu) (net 14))
 (segment (start 128.79102 72.75862) (end 127.1524 71.12) (width 0.25) (layer F.Cu) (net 14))
 (segment (start 127.1524 71.12) (end 127 71.12) (width 0.25) (layer F.Cu) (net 14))
 (segment (start 130.04 76.01) (end 130.04 71.4676) (width 0.25) (layer F.Cu) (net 15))
 (segment (start 130.04 71.4676) (end 127.1524 68.58) (width 0.25) (layer F.Cu) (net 15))
 (segment (start 127.1524 68.58) (end 127 68.58) (width 0.25) (layer F.Cu) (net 15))
 (segment (start 131.89 74.16) (end 131.89 70.7776) (width 0.25) (layer F.Cu) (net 16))
 (segment (start 131.89 70.7776) (end 127.1524 66.04) (width 0.25) (layer F.Cu) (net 16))
 (segment (start 127.1524 66.04) (end 127 66.04) (width 0.25) (layer F.Cu) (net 16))
 (segment (start 132.69 74.16) (end 132.69 69.0376) (width 0.25) (layer F.Cu) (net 17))
 (segment (start 132.69 69.0376) (end 127.1524 63.5) (width 0.25) (layer F.Cu) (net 17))
 (segment (start 127.1524 63.5) (end 127 63.5) (width 0.25) (layer F.Cu) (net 17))
 (segment (start 133.49 74.16) (end 133.49 67.2976) (width 0.25) (layer F.Cu) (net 18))
 (segment (start 133.49 67.2976) (end 127.1524 60.96) (width 0.25) (layer F.Cu) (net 18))
 (segment (start 127.1524 60.96) (end 127 60.96) (width 0.25) (layer F.Cu) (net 18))
 (segment (start 134.29 74.16) (end 134.29 67.31) (width 0.25) (layer F.Cu) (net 19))
 (segment (start 134.29 67.31) (end 134.29 65.5576) (width 0.25) (layer F.Cu) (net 19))
 (segment (start 134.29 65.5576) (end 127.1524 58.42) (width 0.25) (layer F.Cu) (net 19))
 (segment (start 135.09 74.16) (end 135.09 63.8176) (width 0.25) (layer F.Cu) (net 20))
 (segment (start 135.09 63.8176) (end 127.1524 55.88) (width 0.25) (layer F.Cu) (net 20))
 (segment (start 127.1524 55.88) (end 127 55.88) (width 0.25) (layer F.Cu) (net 20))
 (segment (start 136.69 74.16) (end 136.69 63.8176) (width 0.25) (layer F.Cu) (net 21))
 (segment (start 136.69 63.8176) (end 144.6276 55.88) (width 0.25) (layer F.Cu) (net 21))
 (segment (start 144.6276 55.88) (end 144.78 55.88) (width 0.25) (layer F.Cu) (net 21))
 (segment (start 137.49 74.16) (end 137.49 65.5576) (width 0.25) (layer F.Cu) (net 22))
 (segment (start 137.49 65.5576) (end 144.6276 58.42) (width 0.25) (layer F.Cu) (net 22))
 (segment (start 144.6276 58.42) (end 144.78 58.42) (width 0.25) (layer F.Cu) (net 22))
 (segment (start 138.29 74.16) (end 138.29 67.2976) (width 0.25) (layer F.Cu) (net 23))
 (segment (start 138.29 67.2976) (end 144.6276 60.96) (width 0.25) (layer F.Cu) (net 23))
 (segment (start 144.6276 60.96) (end 144.78 60.96) (width 0.25) (layer F.Cu) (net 23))
 (segment (start 139.09 74.16) (end 139.09 69.0376) (width 0.25) (layer F.Cu) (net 24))
 (segment (start 144.6276 63.5) (end 144.78 63.5) (width 0.25) (layer F.Cu) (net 24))
 (segment (start 139.09 69.0376) (end 144.6276 63.5) (width 0.25) (layer F.Cu) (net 24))
 (segment (start 139.89 74.16) (end 139.89 70.7776) (width 0.25) (layer F.Cu) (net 25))
 (segment (start 139.89 70.7776) (end 144.6276 66.04) (width 0.25) (layer F.Cu) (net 25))
 (segment (start 144.6276 66.04) (end 144.78 66.04) (width 0.25) (layer F.Cu) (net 25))
 (segment (start 141.74 76.81) (end 140.69 76.81) (width 0.25) (layer F.Cu) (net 26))
 (segment (start 140.69 76.81) (end 140.614999 76.734999) (width 0.25) (layer F.Cu) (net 26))
 (segment (start 140.614999 76.734999) (end 140.614999 73.451653) (width 0.25) (layer F.Cu) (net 26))
 (segment (start 140.614999 73.451653) (end 144 70.066652) (width 0.25) (layer F.Cu) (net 26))
 (segment (start 144 70.066652) (end 144 69.36) (width 0.25) (layer F.Cu) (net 26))
 (segment (start 144 69.36) (end 144.78 68.58) (width 0.25) (layer F.Cu) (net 26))
 (segment (start 141.74 77.61) (end 142.55359 77.61) (width 0.25) (layer F.Cu) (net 27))
 (segment (start 142.55359 77.61) (end 142.98898 77.17461) (width 0.25) (layer F.Cu) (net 27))
 (segment (start 142.98898 77.17461) (end 142.98898 72.75862) (width 0.25) (layer F.Cu) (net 27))
 (segment (start 142.98898 72.75862) (end 144.6276 71.12) (width 0.25) (layer F.Cu) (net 27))
 (segment (start 144.6276 71.12) (end 144.78 71.12) (width 0.25) (layer F.Cu) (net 27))
 (segment (start 144.78 73.66) (end 144.6276 73.66) (width 0.25) (layer F.Cu) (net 28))
 (segment (start 144.6276 73.66) (end 143.43899 74.84861) (width 0.25) (layer F.Cu) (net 28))
 (segment (start 143.43899 74.84861) (end 143.43899 77.36101) (width 0.25) (layer F.Cu) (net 28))
 (segment (start 143.43899 77.36101) (end 142.98898 77.81102) (width 0.25) (layer F.Cu) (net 28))
 (segment (start 142.98898 77.81102) (end 142.98898 78.21102) (width 0.25) (layer F.Cu) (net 28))
 (segment (start 142.98898 78.21102) (end 142.79 78.41) (width 0.25) (layer F.Cu) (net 28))
 (segment (start 142.79 78.41) (end 141.74 78.41) (width 0.25) (layer F.Cu) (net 28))
 (segment (start 144.135262 77.55139) (end 144.54221 77.55139) (width 0.25) (layer F.Cu) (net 29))
 (segment (start 144.54221 77.55139) (end 144.78 77.3136) (width 0.25) (layer F.Cu) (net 29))
 (segment (start 144.78 77.3136) (end 144.78 76.2) (width 0.25) (layer F.Cu) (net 29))
 (segment (start 144 77.6) (end 144.086652 77.6) (width 0.25) (layer F.Cu) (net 29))
 (segment (start 144.086652 77.6) (end 144.135262 77.55139) (width 0.25) (layer F.Cu) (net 29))
 (segment (start 143.438989 78.161011) (end 144 77.6) (width 0.25) (layer F.Cu) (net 29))
 (segment (start 142.79 79.21) (end 143.438989 78.561011) (width 0.25) (layer F.Cu) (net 29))
 (segment (start 143.438989 78.561011) (end 143.438989 78.161011) (width 0.25) (layer F.Cu) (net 29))
 (segment (start 141.74 79.21) (end 142.79 79.21) (width 0.25) (layer F.Cu) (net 29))
 (segment (start 141.74 80.01) (end 144.6236 80.01) (width 0.25) (layer F.Cu) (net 30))
 (segment (start 144.6236 80.01) (end 144.78 79.8536) (width 0.25) (layer F.Cu) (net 30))
 (segment (start 144.78 79.8536) (end 144.78 78.74) (width 0.25) (layer F.Cu) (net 30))
 (segment (start 141.74 80.81) (end 144.31 80.81) (width 0.25) (layer F.Cu) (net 31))
 (segment (start 144.31 80.81) (end 144.78 81.28) (width 0.25) (layer F.Cu) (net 31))
 (segment (start 141.74 81.61) (end 143.099875 81.61) (width 0.5) (layer F.Cu) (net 32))
 (segment (start 143.099875 81.61) (end 144.78 83.290125) (width 0.5) (layer F.Cu) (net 32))
 (segment (start 144.78 83.290125) (end 144.78 83.82) (width 0.5) (layer F.Cu) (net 32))
 (segment (start 141.74 82.41) (end 142.79 82.41) (width 0.25) (layer F.Cu) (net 33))
 (segment (start 142.79 82.41) (end 143.43899 83.05899) (width 0.25) (layer F.Cu) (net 33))
 (segment (start 143.43899 83.05899) (end 143.43899 85.17139) (width 0.25) (layer F.Cu) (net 33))
 (segment (start 143.43899 85.17139) (end 144.6276 86.36) (width 0.25) (layer F.Cu) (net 33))
 (segment (start 144.6276 86.36) (end 144.78 86.36) (width 0.25) (layer F.Cu) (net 33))
 (segment (start 141.74 83.21) (end 142.79 83.21) (width 0.25) (layer F.Cu) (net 34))
 (segment (start 142.79 83.21) (end 142.98898 83.40898) (width 0.25) (layer F.Cu) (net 34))
 (segment (start 142.98898 83.40898) (end 142.98898 87.26138) (width 0.25) (layer F.Cu) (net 34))
 (segment (start 142.98898 87.26138) (end 144.6276 88.9) (width 0.25) (layer F.Cu) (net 34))
 (segment (start 144.6276 88.9) (end 144.78 88.9) (width 0.25) (layer F.Cu) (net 34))
 (segment (start 141.74 84.01) (end 141.74 88.5524) (width 0.25) (layer F.Cu) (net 35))
 (segment (start 141.74 88.5524) (end 144.6276 91.44) (width 0.25) (layer F.Cu) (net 35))
 (segment (start 144.6276 91.44) (end 144.78 91.44) (width 0.25) (layer F.Cu) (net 35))
 (segment (start 139.89 85.86) (end 139.89 89.2424) (width 0.25) (layer F.Cu) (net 36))
 (segment (start 139.89 89.2424) (end 144.6276 93.98) (width 0.25) (layer F.Cu) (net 36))
 (segment (start 144.6276 93.98) (end 144.78 93.98) (width 0.25) (layer F.Cu) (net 36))
 (segment (start 139.09 85.86) (end 139.09 90.9824) (width 0.25) (layer F.Cu) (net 37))
 (segment (start 139.09 90.9824) (end 144.6276 96.52) (width 0.25) (layer F.Cu) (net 37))
 (segment (start 144.6276 96.52) (end 144.78 96.52) (width 0.25) (layer F.Cu) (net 37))
 (segment (start 138.29 85.86) (end 138.29 92.7224) (width 0.25) (layer F.Cu) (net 38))
 (segment (start 138.29 92.7224) (end 144.6276 99.06) (width 0.25) (layer F.Cu) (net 38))
 (segment (start 144.6276 99.06) (end 144.78 99.06) (width 0.25) (layer F.Cu) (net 38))
 (segment (start 137.49 85.86) (end 137.49 94.4624) (width 0.25) (layer F.Cu) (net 39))
 (segment (start 137.49 94.4624) (end 144.6276 101.6) (width 0.25) (layer F.Cu) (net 39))
 (segment (start 144.6276 101.6) (end 144.78 101.6) (width 0.25) (layer F.Cu) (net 39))
 (segment (start 136.69 85.86) (end 136.69 96.2024) (width 0.25) (layer F.Cu) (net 40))
 (segment (start 136.69 96.2024) (end 144.6276 104.14) (width 0.25) (layer F.Cu) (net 40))
 (segment (start 144.6276 104.14) (end 144.78 104.14) (width 0.25) (layer F.Cu) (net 40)))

